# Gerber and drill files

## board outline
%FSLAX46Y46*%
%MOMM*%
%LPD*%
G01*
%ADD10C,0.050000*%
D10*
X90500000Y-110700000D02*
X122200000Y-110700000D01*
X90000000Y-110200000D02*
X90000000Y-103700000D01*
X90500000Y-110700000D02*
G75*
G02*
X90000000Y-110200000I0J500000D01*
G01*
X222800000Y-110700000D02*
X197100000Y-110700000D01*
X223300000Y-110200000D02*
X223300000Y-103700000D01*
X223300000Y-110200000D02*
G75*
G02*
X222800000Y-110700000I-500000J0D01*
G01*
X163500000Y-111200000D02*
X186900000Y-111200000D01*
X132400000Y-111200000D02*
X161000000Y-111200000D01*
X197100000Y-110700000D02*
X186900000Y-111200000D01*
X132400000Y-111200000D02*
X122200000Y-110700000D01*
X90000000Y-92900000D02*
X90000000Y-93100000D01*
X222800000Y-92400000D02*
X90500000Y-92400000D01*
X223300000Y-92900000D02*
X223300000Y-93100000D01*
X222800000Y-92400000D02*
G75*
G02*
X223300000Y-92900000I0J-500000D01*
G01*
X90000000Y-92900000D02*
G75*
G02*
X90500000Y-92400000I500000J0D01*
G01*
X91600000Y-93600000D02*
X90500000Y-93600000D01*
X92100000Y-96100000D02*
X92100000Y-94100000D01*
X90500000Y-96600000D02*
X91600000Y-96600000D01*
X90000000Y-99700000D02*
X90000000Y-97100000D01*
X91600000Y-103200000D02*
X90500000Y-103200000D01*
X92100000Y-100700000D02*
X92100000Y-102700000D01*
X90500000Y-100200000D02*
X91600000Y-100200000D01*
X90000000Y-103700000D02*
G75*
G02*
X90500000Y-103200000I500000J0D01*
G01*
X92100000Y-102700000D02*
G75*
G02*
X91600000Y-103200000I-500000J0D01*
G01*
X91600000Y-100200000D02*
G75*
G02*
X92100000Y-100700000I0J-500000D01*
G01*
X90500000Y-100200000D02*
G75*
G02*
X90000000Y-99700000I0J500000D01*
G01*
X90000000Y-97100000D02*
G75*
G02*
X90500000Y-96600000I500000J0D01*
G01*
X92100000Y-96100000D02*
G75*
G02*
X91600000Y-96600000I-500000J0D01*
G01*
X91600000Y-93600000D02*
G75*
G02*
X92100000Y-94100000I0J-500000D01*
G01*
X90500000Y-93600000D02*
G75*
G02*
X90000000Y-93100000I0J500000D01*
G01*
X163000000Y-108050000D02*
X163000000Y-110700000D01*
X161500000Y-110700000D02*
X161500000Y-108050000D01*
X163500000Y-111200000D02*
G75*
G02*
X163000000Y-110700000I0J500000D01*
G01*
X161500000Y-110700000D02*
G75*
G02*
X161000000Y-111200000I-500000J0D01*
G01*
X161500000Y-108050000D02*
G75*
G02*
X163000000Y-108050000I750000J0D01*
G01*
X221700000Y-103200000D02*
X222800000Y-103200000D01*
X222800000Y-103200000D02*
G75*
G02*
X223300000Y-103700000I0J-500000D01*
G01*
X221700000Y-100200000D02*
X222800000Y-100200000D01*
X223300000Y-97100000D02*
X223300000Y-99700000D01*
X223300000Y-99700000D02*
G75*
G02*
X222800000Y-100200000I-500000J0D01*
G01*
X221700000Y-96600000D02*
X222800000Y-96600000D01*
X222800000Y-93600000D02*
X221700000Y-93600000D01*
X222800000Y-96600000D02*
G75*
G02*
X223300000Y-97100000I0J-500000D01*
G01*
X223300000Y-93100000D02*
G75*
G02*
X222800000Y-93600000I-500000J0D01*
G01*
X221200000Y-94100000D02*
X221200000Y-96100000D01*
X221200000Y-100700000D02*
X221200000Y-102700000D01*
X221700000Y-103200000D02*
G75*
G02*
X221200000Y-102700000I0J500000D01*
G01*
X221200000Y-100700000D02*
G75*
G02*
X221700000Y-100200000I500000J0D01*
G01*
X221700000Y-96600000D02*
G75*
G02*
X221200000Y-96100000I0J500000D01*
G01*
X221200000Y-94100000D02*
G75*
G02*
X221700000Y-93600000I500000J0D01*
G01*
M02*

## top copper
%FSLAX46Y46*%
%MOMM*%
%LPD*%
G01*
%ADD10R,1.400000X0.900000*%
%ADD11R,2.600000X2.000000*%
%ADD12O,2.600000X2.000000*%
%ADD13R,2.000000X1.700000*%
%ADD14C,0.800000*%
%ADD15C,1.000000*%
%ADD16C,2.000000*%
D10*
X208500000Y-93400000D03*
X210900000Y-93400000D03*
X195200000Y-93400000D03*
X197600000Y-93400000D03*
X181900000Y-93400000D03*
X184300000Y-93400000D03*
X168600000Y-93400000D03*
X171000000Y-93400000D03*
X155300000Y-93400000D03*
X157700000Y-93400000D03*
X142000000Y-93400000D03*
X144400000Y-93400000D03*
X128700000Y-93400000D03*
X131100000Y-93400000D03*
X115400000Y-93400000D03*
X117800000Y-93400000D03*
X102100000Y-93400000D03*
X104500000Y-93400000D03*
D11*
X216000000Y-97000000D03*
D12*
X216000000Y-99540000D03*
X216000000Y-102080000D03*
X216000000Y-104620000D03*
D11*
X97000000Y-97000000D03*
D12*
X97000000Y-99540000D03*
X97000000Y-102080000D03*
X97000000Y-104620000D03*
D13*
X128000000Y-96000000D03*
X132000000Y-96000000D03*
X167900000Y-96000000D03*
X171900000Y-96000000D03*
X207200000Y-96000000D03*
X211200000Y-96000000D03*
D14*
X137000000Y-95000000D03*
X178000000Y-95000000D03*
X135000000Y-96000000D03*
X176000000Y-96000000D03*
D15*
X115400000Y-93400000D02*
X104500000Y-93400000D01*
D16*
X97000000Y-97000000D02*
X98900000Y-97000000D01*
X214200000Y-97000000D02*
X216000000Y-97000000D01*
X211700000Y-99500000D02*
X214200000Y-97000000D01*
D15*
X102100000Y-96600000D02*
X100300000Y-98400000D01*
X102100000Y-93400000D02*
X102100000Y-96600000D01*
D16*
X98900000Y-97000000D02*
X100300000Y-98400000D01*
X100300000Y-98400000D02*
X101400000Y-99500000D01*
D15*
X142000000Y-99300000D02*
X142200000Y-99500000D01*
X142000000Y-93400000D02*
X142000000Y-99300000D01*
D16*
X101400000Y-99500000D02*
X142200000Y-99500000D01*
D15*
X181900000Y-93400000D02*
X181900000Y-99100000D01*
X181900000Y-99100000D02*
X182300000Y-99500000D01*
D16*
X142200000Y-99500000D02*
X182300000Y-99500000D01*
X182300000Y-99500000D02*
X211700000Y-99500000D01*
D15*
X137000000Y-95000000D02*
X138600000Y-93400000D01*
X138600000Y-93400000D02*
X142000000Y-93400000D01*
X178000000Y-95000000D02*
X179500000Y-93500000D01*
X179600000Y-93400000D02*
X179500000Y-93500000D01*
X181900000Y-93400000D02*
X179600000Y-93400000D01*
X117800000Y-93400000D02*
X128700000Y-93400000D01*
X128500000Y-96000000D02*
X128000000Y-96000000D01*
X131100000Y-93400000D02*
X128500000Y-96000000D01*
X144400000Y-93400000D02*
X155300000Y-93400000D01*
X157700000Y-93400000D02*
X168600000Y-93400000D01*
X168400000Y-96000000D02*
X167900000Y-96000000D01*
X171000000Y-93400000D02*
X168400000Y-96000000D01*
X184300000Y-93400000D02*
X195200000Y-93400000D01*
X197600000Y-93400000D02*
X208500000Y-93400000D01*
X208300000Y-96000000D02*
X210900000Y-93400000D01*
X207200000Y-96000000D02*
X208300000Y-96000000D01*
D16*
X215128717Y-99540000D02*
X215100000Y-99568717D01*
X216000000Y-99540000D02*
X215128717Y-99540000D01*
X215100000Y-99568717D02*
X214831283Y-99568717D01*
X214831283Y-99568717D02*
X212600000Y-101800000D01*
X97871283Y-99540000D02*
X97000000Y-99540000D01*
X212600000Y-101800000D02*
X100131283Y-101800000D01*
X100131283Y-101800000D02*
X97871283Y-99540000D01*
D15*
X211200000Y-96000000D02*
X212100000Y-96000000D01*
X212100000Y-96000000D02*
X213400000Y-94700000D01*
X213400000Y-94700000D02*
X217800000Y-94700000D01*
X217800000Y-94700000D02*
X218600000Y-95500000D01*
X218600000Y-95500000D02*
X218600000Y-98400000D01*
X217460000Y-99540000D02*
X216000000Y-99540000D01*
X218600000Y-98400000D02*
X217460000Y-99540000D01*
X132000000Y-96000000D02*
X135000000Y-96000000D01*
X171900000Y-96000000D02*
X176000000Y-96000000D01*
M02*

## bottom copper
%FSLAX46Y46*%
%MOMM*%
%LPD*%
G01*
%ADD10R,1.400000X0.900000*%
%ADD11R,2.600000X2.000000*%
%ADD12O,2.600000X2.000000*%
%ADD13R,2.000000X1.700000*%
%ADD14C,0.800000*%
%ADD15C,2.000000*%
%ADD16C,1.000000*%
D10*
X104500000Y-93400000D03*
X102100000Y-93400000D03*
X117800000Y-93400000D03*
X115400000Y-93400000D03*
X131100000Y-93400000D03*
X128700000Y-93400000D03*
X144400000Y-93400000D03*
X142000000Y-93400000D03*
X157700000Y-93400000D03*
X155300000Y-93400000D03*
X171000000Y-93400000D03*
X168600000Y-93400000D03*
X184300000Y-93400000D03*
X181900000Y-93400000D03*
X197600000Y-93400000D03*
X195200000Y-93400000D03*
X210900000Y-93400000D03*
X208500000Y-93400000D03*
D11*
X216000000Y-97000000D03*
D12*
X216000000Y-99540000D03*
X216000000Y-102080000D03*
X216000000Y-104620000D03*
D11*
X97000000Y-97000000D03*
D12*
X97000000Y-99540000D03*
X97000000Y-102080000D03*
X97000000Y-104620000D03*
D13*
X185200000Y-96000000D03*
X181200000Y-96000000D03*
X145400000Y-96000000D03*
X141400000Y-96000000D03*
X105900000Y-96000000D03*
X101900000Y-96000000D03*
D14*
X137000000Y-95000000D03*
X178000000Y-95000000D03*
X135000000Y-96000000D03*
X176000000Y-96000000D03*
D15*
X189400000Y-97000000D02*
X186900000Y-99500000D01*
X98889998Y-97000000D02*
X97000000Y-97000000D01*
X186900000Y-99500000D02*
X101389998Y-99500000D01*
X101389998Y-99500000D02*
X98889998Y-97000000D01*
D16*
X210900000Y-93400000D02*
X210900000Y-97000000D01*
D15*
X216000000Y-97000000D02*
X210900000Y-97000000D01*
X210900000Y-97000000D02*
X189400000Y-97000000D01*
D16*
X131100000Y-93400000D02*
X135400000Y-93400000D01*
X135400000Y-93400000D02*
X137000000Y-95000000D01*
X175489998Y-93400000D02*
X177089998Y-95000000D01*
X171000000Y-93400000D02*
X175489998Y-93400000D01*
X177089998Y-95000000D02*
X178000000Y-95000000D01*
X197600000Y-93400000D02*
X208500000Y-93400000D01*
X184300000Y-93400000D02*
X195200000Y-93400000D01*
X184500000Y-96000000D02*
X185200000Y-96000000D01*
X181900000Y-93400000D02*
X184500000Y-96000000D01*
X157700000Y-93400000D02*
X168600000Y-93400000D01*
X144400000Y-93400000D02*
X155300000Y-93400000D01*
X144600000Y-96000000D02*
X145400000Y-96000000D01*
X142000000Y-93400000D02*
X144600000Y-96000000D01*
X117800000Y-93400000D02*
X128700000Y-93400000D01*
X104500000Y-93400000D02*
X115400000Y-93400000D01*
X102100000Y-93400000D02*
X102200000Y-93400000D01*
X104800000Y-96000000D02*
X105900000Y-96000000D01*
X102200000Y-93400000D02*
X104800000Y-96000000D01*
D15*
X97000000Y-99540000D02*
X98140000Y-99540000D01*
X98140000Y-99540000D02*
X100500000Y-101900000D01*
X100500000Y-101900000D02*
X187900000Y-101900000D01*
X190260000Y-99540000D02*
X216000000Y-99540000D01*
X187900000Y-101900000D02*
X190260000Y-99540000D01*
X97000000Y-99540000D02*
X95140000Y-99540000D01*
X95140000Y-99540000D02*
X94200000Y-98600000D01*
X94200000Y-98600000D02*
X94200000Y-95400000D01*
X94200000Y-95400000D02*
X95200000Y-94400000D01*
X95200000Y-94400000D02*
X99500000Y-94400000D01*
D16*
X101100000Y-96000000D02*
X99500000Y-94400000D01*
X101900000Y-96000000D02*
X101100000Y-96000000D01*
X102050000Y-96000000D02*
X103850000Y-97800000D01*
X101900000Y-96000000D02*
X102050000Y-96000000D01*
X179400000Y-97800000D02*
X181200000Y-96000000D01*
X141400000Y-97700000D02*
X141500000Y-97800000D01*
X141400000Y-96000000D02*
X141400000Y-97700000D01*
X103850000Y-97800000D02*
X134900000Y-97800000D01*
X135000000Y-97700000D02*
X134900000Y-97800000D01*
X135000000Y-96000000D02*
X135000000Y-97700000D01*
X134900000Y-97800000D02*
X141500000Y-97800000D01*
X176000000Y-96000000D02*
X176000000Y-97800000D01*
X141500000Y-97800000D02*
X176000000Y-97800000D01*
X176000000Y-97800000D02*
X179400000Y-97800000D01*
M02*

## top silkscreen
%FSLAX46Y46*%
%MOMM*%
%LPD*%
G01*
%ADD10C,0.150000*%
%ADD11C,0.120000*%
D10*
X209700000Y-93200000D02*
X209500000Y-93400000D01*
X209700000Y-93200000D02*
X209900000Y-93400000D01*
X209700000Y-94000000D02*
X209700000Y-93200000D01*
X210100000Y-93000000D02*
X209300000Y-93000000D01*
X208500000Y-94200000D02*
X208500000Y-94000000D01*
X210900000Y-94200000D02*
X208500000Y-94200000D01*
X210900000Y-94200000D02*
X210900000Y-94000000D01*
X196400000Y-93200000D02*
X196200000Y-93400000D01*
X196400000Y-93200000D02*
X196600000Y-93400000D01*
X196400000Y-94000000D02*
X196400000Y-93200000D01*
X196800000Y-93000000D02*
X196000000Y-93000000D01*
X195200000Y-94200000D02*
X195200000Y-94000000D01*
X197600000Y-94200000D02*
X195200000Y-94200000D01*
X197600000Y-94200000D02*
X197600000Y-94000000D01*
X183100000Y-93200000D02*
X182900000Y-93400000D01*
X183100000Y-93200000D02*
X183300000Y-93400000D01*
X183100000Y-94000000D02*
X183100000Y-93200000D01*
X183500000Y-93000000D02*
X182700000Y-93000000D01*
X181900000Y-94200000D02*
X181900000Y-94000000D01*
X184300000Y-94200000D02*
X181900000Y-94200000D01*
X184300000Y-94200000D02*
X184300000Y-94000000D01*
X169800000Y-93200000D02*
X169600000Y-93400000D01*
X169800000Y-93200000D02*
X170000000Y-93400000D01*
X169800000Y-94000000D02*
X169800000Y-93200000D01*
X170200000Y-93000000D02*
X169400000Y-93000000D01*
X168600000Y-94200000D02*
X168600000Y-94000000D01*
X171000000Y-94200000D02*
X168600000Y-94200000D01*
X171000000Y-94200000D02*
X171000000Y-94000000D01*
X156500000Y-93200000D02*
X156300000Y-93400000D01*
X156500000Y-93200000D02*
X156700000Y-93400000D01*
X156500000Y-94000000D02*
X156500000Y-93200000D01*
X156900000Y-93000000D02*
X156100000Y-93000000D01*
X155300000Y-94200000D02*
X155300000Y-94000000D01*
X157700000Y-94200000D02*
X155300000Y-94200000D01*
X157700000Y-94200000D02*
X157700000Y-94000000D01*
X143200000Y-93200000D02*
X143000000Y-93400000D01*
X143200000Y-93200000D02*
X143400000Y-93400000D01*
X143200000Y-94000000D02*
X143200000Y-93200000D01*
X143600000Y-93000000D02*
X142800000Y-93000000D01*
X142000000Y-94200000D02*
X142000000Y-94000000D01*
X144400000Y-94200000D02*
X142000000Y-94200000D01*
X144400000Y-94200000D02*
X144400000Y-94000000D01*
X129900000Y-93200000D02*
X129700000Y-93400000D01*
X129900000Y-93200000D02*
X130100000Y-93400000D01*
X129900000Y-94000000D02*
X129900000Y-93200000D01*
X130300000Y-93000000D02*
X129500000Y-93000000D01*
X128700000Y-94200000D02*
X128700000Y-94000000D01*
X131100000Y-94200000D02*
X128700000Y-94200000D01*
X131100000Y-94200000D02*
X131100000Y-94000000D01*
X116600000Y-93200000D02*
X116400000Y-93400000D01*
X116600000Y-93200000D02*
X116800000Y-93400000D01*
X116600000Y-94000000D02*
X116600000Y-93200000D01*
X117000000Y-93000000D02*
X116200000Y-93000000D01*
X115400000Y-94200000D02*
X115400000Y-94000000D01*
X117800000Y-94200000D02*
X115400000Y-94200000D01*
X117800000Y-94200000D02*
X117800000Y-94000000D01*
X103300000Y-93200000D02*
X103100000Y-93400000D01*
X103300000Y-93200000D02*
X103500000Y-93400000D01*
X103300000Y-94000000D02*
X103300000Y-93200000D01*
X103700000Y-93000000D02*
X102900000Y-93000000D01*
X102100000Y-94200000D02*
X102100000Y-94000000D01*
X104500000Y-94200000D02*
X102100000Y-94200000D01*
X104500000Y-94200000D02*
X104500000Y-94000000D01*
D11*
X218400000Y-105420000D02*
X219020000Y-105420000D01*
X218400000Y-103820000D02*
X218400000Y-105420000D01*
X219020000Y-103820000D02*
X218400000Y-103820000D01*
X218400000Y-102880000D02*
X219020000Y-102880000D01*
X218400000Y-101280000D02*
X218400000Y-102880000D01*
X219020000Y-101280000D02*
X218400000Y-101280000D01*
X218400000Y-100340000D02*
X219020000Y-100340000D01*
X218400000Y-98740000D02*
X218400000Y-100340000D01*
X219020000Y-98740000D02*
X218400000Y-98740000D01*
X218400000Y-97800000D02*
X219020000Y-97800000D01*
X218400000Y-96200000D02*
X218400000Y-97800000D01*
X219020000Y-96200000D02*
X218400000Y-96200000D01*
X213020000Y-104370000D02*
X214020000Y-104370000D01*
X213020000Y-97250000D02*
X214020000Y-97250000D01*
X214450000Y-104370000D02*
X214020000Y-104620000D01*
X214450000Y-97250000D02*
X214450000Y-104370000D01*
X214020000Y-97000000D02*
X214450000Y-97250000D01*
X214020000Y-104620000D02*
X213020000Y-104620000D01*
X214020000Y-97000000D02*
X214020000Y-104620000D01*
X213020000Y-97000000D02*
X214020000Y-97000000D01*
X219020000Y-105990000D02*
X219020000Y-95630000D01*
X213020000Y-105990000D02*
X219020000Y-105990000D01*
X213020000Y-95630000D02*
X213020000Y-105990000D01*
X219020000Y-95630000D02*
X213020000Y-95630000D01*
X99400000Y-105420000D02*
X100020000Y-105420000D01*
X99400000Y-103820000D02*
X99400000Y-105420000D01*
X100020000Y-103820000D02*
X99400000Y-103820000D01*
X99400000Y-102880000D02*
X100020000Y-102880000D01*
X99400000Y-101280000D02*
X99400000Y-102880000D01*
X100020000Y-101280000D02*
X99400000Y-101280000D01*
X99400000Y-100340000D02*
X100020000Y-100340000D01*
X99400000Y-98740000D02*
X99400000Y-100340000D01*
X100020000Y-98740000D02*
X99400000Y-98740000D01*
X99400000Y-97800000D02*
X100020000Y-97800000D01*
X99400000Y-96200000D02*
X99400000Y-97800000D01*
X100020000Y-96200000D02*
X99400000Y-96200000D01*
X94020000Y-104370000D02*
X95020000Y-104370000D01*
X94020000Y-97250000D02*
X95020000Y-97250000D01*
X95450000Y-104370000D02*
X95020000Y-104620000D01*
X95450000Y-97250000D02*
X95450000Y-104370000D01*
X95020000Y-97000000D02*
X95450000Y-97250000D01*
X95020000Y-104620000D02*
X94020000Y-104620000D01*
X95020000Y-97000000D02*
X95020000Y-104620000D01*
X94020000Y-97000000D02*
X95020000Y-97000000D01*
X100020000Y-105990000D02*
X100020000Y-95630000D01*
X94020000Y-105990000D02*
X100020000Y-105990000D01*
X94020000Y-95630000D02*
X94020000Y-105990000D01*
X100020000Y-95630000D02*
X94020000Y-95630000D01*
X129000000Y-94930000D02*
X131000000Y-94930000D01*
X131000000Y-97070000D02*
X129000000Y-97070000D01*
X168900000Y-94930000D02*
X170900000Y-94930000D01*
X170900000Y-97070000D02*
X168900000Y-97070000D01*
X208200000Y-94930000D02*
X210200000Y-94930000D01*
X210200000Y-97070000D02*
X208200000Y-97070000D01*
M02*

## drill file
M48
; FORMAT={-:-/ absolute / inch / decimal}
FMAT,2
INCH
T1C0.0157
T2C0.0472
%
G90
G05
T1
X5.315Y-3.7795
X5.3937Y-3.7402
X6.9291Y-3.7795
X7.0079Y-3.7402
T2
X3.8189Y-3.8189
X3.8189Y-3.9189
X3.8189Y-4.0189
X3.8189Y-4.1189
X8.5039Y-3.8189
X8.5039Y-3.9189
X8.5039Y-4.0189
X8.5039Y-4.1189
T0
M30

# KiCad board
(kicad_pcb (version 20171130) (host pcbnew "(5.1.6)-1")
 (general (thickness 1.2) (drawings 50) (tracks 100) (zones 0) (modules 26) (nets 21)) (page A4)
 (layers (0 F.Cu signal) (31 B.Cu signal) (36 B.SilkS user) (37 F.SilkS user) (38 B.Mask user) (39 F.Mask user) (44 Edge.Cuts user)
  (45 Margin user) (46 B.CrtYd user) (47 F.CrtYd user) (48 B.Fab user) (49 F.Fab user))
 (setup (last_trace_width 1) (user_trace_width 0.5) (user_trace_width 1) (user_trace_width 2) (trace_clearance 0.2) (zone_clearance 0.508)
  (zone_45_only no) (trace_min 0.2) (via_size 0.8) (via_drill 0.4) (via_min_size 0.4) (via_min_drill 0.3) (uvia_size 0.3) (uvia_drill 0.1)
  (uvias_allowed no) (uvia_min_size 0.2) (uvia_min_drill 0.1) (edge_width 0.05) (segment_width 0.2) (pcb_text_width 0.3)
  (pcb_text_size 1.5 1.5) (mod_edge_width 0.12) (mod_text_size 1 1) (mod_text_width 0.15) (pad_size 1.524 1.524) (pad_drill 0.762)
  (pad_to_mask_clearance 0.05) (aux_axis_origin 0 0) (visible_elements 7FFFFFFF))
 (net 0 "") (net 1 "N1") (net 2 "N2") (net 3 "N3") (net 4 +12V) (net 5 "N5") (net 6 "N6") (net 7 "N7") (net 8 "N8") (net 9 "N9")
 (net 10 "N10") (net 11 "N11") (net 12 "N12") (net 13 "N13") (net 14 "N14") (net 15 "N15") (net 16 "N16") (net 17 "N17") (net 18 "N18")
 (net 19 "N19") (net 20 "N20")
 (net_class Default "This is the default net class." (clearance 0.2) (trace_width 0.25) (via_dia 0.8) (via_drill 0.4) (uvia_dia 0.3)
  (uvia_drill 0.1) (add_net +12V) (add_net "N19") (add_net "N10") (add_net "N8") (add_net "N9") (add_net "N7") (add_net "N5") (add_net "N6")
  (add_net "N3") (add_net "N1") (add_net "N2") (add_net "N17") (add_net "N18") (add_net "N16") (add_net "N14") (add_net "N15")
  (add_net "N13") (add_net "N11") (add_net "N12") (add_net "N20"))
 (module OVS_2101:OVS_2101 (layer B.Cu) (at 103.3 93.4)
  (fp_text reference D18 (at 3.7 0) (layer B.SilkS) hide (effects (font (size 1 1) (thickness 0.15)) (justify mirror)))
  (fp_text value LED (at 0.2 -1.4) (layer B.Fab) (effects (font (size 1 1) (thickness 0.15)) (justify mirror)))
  (pad 2 smd rect (at 1.2 0) (size 1.4 0.9) (layers B.Cu B.Paste B.Mask) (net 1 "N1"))
  (pad 1 smd rect (at -1.2 0) (size 1.4 0.9) (layers B.Cu B.Paste B.Mask) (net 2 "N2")))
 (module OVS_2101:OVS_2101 (layer B.Cu) (at 116.6 93.4)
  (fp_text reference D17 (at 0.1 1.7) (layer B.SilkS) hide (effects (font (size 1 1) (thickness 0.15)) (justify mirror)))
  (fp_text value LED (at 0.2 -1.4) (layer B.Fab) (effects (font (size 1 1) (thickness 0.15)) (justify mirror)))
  (pad 2 smd rect (at 1.2 0) (size 1.4 0.9) (layers B.Cu B.Paste B.Mask) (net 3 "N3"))
  (pad 1 smd rect (at -1.2 0) (size 1.4 0.9) (layers B.Cu B.Paste B.Mask) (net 1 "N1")))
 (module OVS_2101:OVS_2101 (layer B.Cu) (at 129.9 93.4)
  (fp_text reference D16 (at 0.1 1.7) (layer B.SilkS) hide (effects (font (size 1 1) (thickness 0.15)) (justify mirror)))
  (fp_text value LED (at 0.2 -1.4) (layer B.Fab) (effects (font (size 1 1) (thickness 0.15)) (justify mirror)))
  (pad 2 smd rect (at 1.2 0) (size 1.4 0.9) (layers B.Cu B.Paste B.Mask) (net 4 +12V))
  (pad 1 smd rect (at -1.2 0) (size 1.4 0.9) (layers B.Cu B.Paste B.Mask) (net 3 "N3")))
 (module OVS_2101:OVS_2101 (layer B.Cu) (at 143.2 93.4)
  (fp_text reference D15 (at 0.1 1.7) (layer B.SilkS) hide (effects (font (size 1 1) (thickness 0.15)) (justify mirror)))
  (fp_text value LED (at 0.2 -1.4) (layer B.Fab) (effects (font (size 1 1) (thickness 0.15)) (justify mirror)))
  (pad 2 smd rect (at 1.2 0) (size 1.4 0.9) (layers B.Cu B.Paste B.Mask) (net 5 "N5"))
  (pad 1 smd rect (at -1.2 0) (size 1.4 0.9) (layers B.Cu B.Paste B.Mask) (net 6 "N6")))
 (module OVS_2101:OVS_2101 (layer B.Cu) (at 156.5 93.4)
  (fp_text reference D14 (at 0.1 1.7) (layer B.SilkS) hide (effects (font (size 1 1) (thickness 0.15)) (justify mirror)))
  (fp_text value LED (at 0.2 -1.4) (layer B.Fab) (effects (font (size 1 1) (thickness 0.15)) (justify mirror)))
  (pad 2 smd rect (at 1.2 0) (size 1.4 0.9) (layers B.Cu B.Paste B.Mask) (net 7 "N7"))
  (pad 1 smd rect (at -1.2 0) (size 1.4 0.9) (layers B.Cu B.Paste B.Mask) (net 5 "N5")))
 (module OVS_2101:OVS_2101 (layer B.Cu) (at 169.8 93.4)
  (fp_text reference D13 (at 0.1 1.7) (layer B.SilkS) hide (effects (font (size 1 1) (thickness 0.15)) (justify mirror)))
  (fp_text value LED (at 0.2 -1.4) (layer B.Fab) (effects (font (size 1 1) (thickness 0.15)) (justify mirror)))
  (pad 2 smd rect (at 1.2 0) (size 1.4 0.9) (layers B.Cu B.Paste B.Mask) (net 4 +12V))
  (pad 1 smd rect (at -1.2 0) (size 1.4 0.9) (layers B.Cu B.Paste B.Mask) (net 7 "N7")))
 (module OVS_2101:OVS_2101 (layer B.Cu) (at 183.1 93.4)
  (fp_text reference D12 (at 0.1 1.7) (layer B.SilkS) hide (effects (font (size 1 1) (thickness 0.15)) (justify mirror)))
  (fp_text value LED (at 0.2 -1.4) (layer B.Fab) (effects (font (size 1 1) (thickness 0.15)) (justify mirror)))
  (pad 2 smd rect (at 1.2 0) (size 1.4 0.9) (layers B.Cu B.Paste B.Mask) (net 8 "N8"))
  (pad 1 smd rect (at -1.2 0) (size 1.4 0.9) (layers B.Cu B.Paste B.Mask) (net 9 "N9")))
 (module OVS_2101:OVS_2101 (layer B.Cu) (at 196.4 93.4)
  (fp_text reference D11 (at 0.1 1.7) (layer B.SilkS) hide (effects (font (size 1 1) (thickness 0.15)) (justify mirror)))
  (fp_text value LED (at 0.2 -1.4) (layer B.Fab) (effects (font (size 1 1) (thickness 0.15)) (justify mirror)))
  (pad 2 smd rect (at 1.2 0) (size 1.4 0.9) (layers B.Cu B.Paste B.Mask) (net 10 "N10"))
  (pad 1 smd rect (at -1.2 0) (size 1.4 0.9) (layers B.Cu B.Paste B.Mask) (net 8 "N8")))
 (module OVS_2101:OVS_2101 (layer B.Cu) (at 209.7 93.4)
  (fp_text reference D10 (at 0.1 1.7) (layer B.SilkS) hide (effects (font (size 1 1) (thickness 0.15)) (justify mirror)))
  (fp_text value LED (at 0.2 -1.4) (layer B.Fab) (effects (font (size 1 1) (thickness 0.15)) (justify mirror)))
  (pad 2 smd rect (at 1.2 0) (size 1.4 0.9) (layers B.Cu B.Paste B.Mask) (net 4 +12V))
  (pad 1 smd rect (at -1.2 0) (size 1.4 0.9) (layers B.Cu B.Paste B.Mask) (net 10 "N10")))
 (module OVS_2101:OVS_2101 (layer F.Cu) (at 209.7 93.4 180)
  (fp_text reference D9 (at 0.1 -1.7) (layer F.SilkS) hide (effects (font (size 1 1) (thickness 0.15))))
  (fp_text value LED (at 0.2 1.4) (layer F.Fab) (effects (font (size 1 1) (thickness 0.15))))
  (fp_line (start 0 0.2) (end 0.2 0) (layer F.SilkS) (width 0.15))
  (fp_line (start 0 0.2) (end -0.2 0) (layer F.SilkS) (width 0.15))
  (fp_line (start 0 -0.6) (end 0 0.2) (layer F.SilkS) (width 0.15))
  (fp_line (start -0.4 0.4) (end 0.4 0.4) (layer F.SilkS) (width 0.15))
  (fp_line (start 1.2 -0.8) (end 1.2 -0.6) (layer F.SilkS) (width 0.15))
  (fp_line (start -1.2 -0.8) (end 1.2 -0.8) (layer F.SilkS) (width 0.15))
  (fp_line (start -1.2 -0.8) (end -1.2 -0.6) (layer F.SilkS) (width 0.15))
  (pad 2 smd rect (at 1.2 0 180) (size 1.4 0.9) (layers F.Cu F.Paste F.Mask) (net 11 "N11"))
  (pad 1 smd rect (at -1.2 0 180) (size 1.4 0.9) (layers F.Cu F.Paste F.Mask) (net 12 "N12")))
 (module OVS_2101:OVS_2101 (layer F.Cu) (at 196.4 93.4 180)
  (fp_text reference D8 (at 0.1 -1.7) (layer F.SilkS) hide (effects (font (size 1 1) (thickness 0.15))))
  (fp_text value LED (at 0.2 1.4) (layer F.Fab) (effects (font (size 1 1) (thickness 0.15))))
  (fp_line (start 0 0.2) (end 0.2 0) (layer F.SilkS) (width 0.15))
  (fp_line (start 0 0.2) (end -0.2 0) (layer F.SilkS) (width 0.15))
  (fp_line (start 0 -0.6) (end 0 0.2) (layer F.SilkS) (width 0.15))
  (fp_line (start -0.4 0.4) (end 0.4 0.4) (layer F.SilkS) (width 0.15))
  (fp_line (start 1.2 -0.8) (end 1.2 -0.6) (layer F.SilkS) (width 0.15))
  (fp_line (start -1.2 -0.8) (end 1.2 -0.8) (layer F.SilkS) (width 0.15))
  (fp_line (start -1.2 -0.8) (end -1.2 -0.6) (layer F.SilkS) (width 0.15))
  (pad 2 smd rect (at 1.2 0 180) (size 1.4 0.9) (layers F.Cu F.Paste F.Mask) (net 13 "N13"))
  (pad 1 smd rect (at -1.2 0 180) (size 1.4 0.9) (layers F.Cu F.Paste F.Mask) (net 11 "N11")))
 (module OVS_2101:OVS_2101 (layer F.Cu) (at 183.1 93.4 180)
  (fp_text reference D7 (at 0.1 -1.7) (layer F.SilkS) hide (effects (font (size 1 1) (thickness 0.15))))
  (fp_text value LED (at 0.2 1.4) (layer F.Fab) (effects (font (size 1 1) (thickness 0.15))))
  (fp_line (start 0 0.2) (end 0.2 0) (layer F.SilkS) (width 0.15))
  (fp_line (start 0 0.2) (end -0.2 0) (layer F.SilkS) (width 0.15))
  (fp_line (start 0 -0.6) (end 0 0.2) (layer F.SilkS) (width 0.15))
  (fp_line (start -0.4 0.4) (end 0.4 0.4) (layer F.SilkS) (width 0.15))
  (fp_line (start 1.2 -0.8) (end 1.2 -0.6) (layer F.SilkS) (width 0.15))
  (fp_line (start -1.2 -0.8) (end 1.2 -0.8) (layer F.SilkS) (width 0.15))
  (fp_line (start -1.2 -0.8) (end -1.2 -0.6) (layer F.SilkS) (width 0.15))
  (pad 2 smd rect (at 1.2 0 180) (size 1.4 0.9) (layers F.Cu F.Paste F.Mask) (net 4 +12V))
  (pad 1 smd rect (at -1.2 0 180) (size 1.4 0.9) (layers F.Cu F.Paste F.Mask) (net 13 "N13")))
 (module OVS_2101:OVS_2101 (layer F.Cu) (at 169.8 93.4 180)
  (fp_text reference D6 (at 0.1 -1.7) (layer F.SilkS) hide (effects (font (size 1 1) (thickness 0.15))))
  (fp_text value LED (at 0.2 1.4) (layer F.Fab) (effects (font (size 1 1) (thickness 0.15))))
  (fp_line (start 0 0.2) (end 0.2 0) (layer F.SilkS) (width 0.15))
  (fp_line (start 0 0.2) (end -0.2 0) (layer F.SilkS) (width 0.15))
  (fp_line (start 0 -0.6) (end 0 0.2) (layer F.SilkS) (width 0.15))
  (fp_line (start -0.4 0.4) (end 0.4 0.4) (layer F.SilkS) (width 0.15))
  (fp_line (start 1.2 -0.8) (end 1.2 -0.6) (layer F.SilkS) (width 0.15))
  (fp_line (start -1.2 -0.8) (end 1.2 -0.8) (layer F.SilkS) (width 0.15))
  (fp_line (start -1.2 -0.8) (end -1.2 -0.6) (layer F.SilkS) (width 0.15))
  (pad 2 smd rect (at 1.2 0 180) (size 1.4 0.9) (layers F.Cu F.Paste F.Mask) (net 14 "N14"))
  (pad 1 smd rect (at -1.2 0 180) (size 1.4 0.9) (layers F.Cu F.Paste F.Mask) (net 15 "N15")))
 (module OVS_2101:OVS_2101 (layer F.Cu) (at 156.5 93.4 180)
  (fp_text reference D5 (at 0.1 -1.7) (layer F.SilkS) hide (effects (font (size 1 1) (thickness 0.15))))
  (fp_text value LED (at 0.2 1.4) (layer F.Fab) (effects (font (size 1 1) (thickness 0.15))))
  (fp_line (start 0 0.2) (end 0.2 0) (layer F.SilkS) (width 0.15))
  (fp_line (start 0 0.2) (end -0.2 0) (layer F.SilkS) (width 0.15))
  (fp_line (start 0 -0.6) (end 0 0.2) (layer F.SilkS) (width 0.15))
  (fp_line (start -0.4 0.4) (end 0.4 0.4) (layer F.SilkS) (width 0.15))
  (fp_line (start 1.2 -0.8) (end 1.2 -0.6) (layer F.SilkS) (width 0.15))
  (fp_line (start -1.2 -0.8) (end 1.2 -0.8) (layer F.SilkS) (width 0.15))
  (fp_line (start -1.2 -0.8) (end -1.2 -0.6) (layer F.SilkS) (width 0.15))
  (pad 2 smd rect (at 1.2 0 180) (size 1.4 0.9) (layers F.Cu F.Paste F.Mask) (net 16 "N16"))
  (pad 1 smd rect (at -1.2 0 180) (size 1.4 0.9) (layers F.Cu F.Paste F.Mask) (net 14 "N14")))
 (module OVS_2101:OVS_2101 (layer F.Cu) (at 143.2 93.4 180)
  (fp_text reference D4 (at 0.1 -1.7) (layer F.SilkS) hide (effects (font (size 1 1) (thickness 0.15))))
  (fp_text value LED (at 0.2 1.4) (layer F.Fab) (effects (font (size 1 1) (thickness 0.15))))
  (fp_line (start 0 0.2) (end 0.2 0) (layer F.SilkS) (width 0.15))
  (fp_line (start 0 0.2) (end -0.2 0) (layer F.SilkS) (width 0.15))
  (fp_line (start 0 -0.6) (end 0 0.2) (layer F.SilkS) (width 0.15))
  (fp_line (start -0.4 0.4) (end 0.4 0.4) (layer F.SilkS) (width 0.15))
  (fp_line (start 1.2 -0.8) (end 1.2 -0.6) (layer F.SilkS) (width 0.15))
  (fp_line (start -1.2 -0.8) (end 1.2 -0.8) (layer F.SilkS) (width 0.15))
  (fp_line (start -1.2 -0.8) (end -1.2 -0.6) (layer F.SilkS) (width 0.15))
  (pad 2 smd rect (at 1.2 0 180) (size 1.4 0.9) (layers F.Cu F.Paste F.Mask) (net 4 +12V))
  (pad 1 smd rect (at -1.2 0 180) (size 1.4 0.9) (layers F.Cu F.Paste F.Mask) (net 16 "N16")))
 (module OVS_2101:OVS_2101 (layer F.Cu) (at 129.9 93.4 180)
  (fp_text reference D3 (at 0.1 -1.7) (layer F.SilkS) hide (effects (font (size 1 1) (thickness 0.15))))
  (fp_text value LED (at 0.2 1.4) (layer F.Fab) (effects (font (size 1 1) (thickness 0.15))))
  (fp_line (start 0 0.2) (end 0.2 0) (layer F.SilkS) (width 0.15))
  (fp_line (start 0 0.2) (end -0.2 0) (layer F.SilkS) (width 0.15))
  (fp_line (start 0 -0.6) (end 0 0.2) (layer F.SilkS) (width 0.15))
  (fp_line (start -0.4 0.4) (end 0.4 0.4) (layer F.SilkS) (width 0.15))
  (fp_line (start 1.2 -0.8) (end 1.2 -0.6) (layer F.SilkS) (width 0.15))
  (fp_line (start -1.2 -0.8) (end 1.2 -0.8) (layer F.SilkS) (width 0.15))
  (fp_line (start -1.2 -0.8) (end -1.2 -0.6) (layer F.SilkS) (width 0.15))
  (pad 2 smd rect (at 1.2 0 180) (size 1.4 0.9) (layers F.Cu F.Paste F.Mask) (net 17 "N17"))
  (pad 1 smd rect (at -1.2 0 180) (size 1.4 0.9) (layers F.Cu F.Paste F.Mask) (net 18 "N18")))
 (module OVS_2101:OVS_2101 (layer F.Cu) (at 116.6 93.4 180)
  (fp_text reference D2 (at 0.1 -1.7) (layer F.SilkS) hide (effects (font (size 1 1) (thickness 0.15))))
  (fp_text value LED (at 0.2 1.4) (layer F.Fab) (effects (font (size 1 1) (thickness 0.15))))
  (fp_line (start 0 0.2) (end 0.2 0) (layer F.SilkS) (width 0.15))
  (fp_line (start 0 0.2) (end -0.2 0) (layer F.SilkS) (width 0.15))
  (fp_line (start 0 -0.6) (end 0 0.2) (layer F.SilkS) (width 0.15))
  (fp_line (start -0.4 0.4) (end 0.4 0.4) (layer F.SilkS) (width 0.15))
  (fp_line (start 1.2 -0.8) (end 1.2 -0.6) (layer F.SilkS) (width 0.15))
  (fp_line (start -1.2 -0.8) (end 1.2 -0.8) (layer F.SilkS) (width 0.15))
  (fp_line (start -1.2 -0.8) (end -1.2 -0.6) (layer F.SilkS) (width 0.15))
  (pad 2 smd rect (at 1.2 0 180) (size 1.4 0.9) (layers F.Cu F.Paste F.Mask) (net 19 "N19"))
  (pad 1 smd rect (at -1.2 0 180) (size 1.4 0.9) (layers F.Cu F.Paste F.Mask) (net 17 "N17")))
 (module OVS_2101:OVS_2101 (layer F.Cu) (at 103.3 93.4 180)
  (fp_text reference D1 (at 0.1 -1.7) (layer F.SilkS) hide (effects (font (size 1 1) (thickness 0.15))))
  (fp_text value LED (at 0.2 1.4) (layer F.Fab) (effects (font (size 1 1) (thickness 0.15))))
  (fp_line (start 0 0.2) (end 0.2 0) (layer F.SilkS) (width 0.15))
  (fp_line (start 0 0.2) (end -0.2 0) (layer F.SilkS) (width 0.15))
  (fp_line (start 0 -0.6) (end 0 0.2) (layer F.SilkS) (width 0.15))
  (fp_line (start -0.4 0.4) (end 0.4 0.4) (layer F.SilkS) (width 0.15))
  (fp_line (start 1.2 -0.8) (end 1.2 -0.6) (layer F.SilkS) (width 0.15))
  (fp_line (start -1.2 -0.8) (end 1.2 -0.8) (layer F.SilkS) (width 0.15))
  (fp_line (start -1.2 -0.8) (end -1.2 -0.6) (layer F.SilkS) (width 0.15))
  (pad 2 smd rect (at 1.2 0 180) (size 1.4 0.9) (layers F.Cu F.Paste F.Mask) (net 4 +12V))
  (pad 1 smd rect (at -1.2 0 180) (size 1.4 0.9) (layers F.Cu F.Paste F.Mask) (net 19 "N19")))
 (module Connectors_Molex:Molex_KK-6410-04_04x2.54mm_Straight (layer F.Cu) (at 216 97 270)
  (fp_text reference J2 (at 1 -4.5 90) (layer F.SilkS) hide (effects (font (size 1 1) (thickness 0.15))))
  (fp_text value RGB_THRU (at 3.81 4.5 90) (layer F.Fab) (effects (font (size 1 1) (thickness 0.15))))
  (fp_line (start 8.42 -2.4) (end 8.42 -3.02) (layer F.SilkS) (width 0.12))
  (fp_line (start 6.82 -2.4) (end 8.42 -2.4) (layer F.SilkS) (width 0.12))
  (fp_line (start 6.82 -3.02) (end 6.82 -2.4) (layer F.SilkS) (width 0.12))
  (fp_line (start 5.88 -2.4) (end 5.88 -3.02) (layer F.SilkS) (width 0.12))
  (fp_line (start 4.28 -2.4) (end 5.88 -2.4) (layer F.SilkS) (width 0.12))
  (fp_line (start 4.28 -3.02) (end 4.28 -2.4) (layer F.SilkS) (width 0.12))
  (fp_line (start 3.34 -2.4) (end 3.34 -3.02) (layer F.SilkS) (width 0.12))
  (fp_line (start 1.74 -2.4) (end 3.34 -2.4) (layer F.SilkS) (width 0.12))
  (fp_line (start 1.74 -3.02) (end 1.74 -2.4) (layer F.SilkS) (width 0.12))
  (fp_line (start 0.8 -2.4) (end 0.8 -3.02) (layer F.SilkS) (width 0.12))
  (fp_line (start -0.8 -2.4) (end 0.8 -2.4) (layer F.SilkS) (width 0.12))
  (fp_line (start -0.8 -3.02) (end -0.8 -2.4) (layer F.SilkS) (width 0.12))
  (fp_line (start 7.37 2.98) (end 7.37 1.98) (layer F.SilkS) (width 0.12))
  (fp_line (start 0.25 2.98) (end 0.25 1.98) (layer F.SilkS) (width 0.12))
  (fp_line (start 7.37 1.55) (end 7.62 1.98) (layer F.SilkS) (width 0.12))
  (fp_line (start 0.25 1.55) (end 7.37 1.55) (layer F.SilkS) (width 0.12))
  (fp_line (start 0 1.98) (end 0.25 1.55) (layer F.SilkS) (width 0.12))
  (fp_line (start 7.62 1.98) (end 7.62 2.98) (layer F.SilkS) (width 0.12))
  (fp_line (start 0 1.98) (end 7.62 1.98) (layer F.SilkS) (width 0.12))
  (fp_line (start 0 2.98) (end 0 1.98) (layer F.SilkS) (width 0.12))
  (fp_line (start 8.99 -3.02) (end -1.37 -3.02) (layer F.SilkS) (width 0.12))
  (fp_line (start 8.99 2.98) (end 8.99 -3.02) (layer F.SilkS) (width 0.12))
  (fp_line (start -1.37 2.98) (end 8.99 2.98) (layer F.SilkS) (width 0.12))
  (fp_line (start -1.37 -3.02) (end -1.37 2.98) (layer F.SilkS) (width 0.12))
  (pad 1 thru_hole rect (at 0 0 270) (size 2 2.6) (drill 1.2) (layers *.Cu *.Mask) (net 4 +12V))
  (pad 2 thru_hole oval (at 2.54 0 270) (size 2 2.6) (drill 1.2) (layers *.Cu *.Mask) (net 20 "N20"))
  (pad 3 thru_hole oval (at 5.08 0 270) (size 2 2.6) (drill 1.2) (layers *.Cu *.Mask))
  (pad 4 thru_hole oval (at 7.62 0 270) (size 2 2.6) (drill 1.2) (layers *.Cu *.Mask)))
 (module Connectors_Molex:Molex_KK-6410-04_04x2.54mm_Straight (layer F.Cu) (at 97 97 270)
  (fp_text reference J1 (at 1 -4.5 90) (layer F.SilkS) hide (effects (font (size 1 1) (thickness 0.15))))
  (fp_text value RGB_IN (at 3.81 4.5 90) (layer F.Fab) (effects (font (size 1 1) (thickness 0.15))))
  (fp_line (start 8.42 -2.4) (end 8.42 -3.02) (layer F.SilkS) (width 0.12))
  (fp_line (start 6.82 -2.4) (end 8.42 -2.4) (layer F.SilkS) (width 0.12))
  (fp_line (start 6.82 -3.02) (end 6.82 -2.4) (layer F.SilkS) (width 0.12))
  (fp_line (start 5.88 -2.4) (end 5.88 -3.02) (layer F.SilkS) (width 0.12))
  (fp_line (start 4.28 -2.4) (end 5.88 -2.4) (layer F.SilkS) (width 0.12))
  (fp_line (start 4.28 -3.02) (end 4.28 -2.4) (layer F.SilkS) (width 0.12))
  (fp_line (start 3.34 -2.4) (end 3.34 -3.02) (layer F.SilkS) (width 0.12))
  (fp_line (start 1.74 -2.4) (end 3.34 -2.4) (layer F.SilkS) (width 0.12))
  (fp_line (start 1.74 -3.02) (end 1.74 -2.4) (layer F.SilkS) (width 0.12))
  (fp_line (start 0.8 -2.4) (end 0.8 -3.02) (layer F.SilkS) (width 0.12))
  (fp_line (start -0.8 -2.4) (end 0.8 -2.4) (layer F.SilkS) (width 0.12))
  (fp_line (start -0.8 -3.02) (end -0.8 -2.4) (layer F.SilkS) (width 0.12))
  (fp_line (start 7.37 2.98) (end 7.37 1.98) (layer F.SilkS) (width 0.12))
  (fp_line (start 0.25 2.98) (end 0.25 1.98) (layer F.SilkS) (width 0.12))
  (fp_line (start 7.37 1.55) (end 7.62 1.98) (layer F.SilkS) (width 0.12))
  (fp_line (start 0.25 1.55) (end 7.37 1.55) (layer F.SilkS) (width 0.12))
  (fp_line (start 0 1.98) (end 0.25 1.55) (layer F.SilkS) (width 0.12))
  (fp_line (start 7.62 1.98) (end 7.62 2.98) (layer F.SilkS) (width 0.12))
  (fp_line (start 0 1.98) (end 7.62 1.98) (layer F.SilkS) (width 0.12))
  (fp_line (start 0 2.98) (end 0 1.98) (layer F.SilkS) (width 0.12))
  (fp_line (start 8.99 -3.02) (end -1.37 -3.02) (layer F.SilkS) (width 0.12))
  (fp_line (start 8.99 2.98) (end 8.99 -3.02) (layer F.SilkS) (width 0.12))
  (fp_line (start -1.37 2.98) (end 8.99 2.98) (layer F.SilkS) (width 0.12))
  (fp_line (start -1.37 -3.02) (end -1.37 2.98) (layer F.SilkS) (width 0.12))
  (pad 1 thru_hole rect (at 0 0 270) (size 2 2.6) (drill 1.2) (layers *.Cu *.Mask) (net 4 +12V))
  (pad 2 thru_hole oval (at 2.54 0 270) (size 2 2.6) (drill 1.2) (layers *.Cu *.Mask) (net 20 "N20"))
  (pad 3 thru_hole oval (at 5.08 0 270) (size 2 2.6) (drill 1.2) (layers *.Cu *.Mask))
  (pad 4 thru_hole oval (at 7.62 0 270) (size 2 2.6) (drill 1.2) (layers *.Cu *.Mask)))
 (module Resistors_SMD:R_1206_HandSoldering (layer F.Cu) (at 130 96)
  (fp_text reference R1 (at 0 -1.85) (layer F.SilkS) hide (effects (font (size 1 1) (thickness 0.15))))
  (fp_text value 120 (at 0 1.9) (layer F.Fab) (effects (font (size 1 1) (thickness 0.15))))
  (fp_line (start -1 -1.07) (end 1 -1.07) (layer F.SilkS) (width 0.12))
  (fp_line (start 1 1.07) (end -1 1.07) (layer F.SilkS) (width 0.12))
  (pad 1 smd rect (at -2 0) (size 2 1.7) (layers F.Cu F.Paste F.Mask) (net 18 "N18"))
  (pad 2 smd rect (at 2 0) (size 2 1.7) (layers F.Cu F.Paste F.Mask) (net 20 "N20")))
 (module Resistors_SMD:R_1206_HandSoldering (layer F.Cu) (at 169.9 96)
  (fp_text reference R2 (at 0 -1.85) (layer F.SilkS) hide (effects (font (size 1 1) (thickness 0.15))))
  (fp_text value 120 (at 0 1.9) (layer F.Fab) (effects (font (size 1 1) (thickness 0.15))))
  (fp_line (start -1 -1.07) (end 1 -1.07) (layer F.SilkS) (width 0.12))
  (fp_line (start 1 1.07) (end -1 1.07) (layer F.SilkS) (width 0.12))
  (pad 1 smd rect (at -2 0) (size 2 1.7) (layers F.Cu F.Paste F.Mask) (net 15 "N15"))
  (pad 2 smd rect (at 2 0) (size 2 1.7) (layers F.Cu F.Paste F.Mask) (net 20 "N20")))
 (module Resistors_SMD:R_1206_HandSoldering (layer F.Cu) (at 209.2 96)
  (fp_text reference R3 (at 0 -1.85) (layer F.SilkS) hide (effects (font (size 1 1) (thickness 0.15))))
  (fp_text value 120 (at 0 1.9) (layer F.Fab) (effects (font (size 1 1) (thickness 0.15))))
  (fp_line (start -1 -1.07) (end 1 -1.07) (layer F.SilkS) (width 0.12))
  (fp_line (start 1 1.07) (end -1 1.07) (layer F.SilkS) (width 0.12))
  (pad 1 smd rect (at -2 0) (size 2 1.7) (layers F.Cu F.Paste F.Mask) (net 12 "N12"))
  (pad 2 smd rect (at 2 0) (size 2 1.7) (layers F.Cu F.Paste F.Mask) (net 20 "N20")))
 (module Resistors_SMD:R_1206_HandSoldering (layer B.Cu) (at 183.2 96 180)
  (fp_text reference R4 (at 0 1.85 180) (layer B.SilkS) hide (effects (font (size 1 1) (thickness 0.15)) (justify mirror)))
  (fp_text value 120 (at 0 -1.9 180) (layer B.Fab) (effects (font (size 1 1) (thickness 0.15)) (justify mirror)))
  (pad 1 smd rect (at -2 0 180) (size 2 1.7) (layers B.Cu B.Paste B.Mask) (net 9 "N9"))
  (pad 2 smd rect (at 2 0 180) (size 2 1.7) (layers B.Cu B.Paste B.Mask) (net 20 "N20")))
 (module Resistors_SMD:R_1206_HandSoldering (layer B.Cu) (at 143.4 96 180)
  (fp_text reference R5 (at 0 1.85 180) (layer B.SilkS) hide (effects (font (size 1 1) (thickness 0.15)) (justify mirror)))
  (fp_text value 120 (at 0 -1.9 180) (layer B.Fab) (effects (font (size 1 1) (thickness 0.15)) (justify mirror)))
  (pad 1 smd rect (at -2 0 180) (size 2 1.7) (layers B.Cu B.Paste B.Mask) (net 6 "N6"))
  (pad 2 smd rect (at 2 0 180) (size 2 1.7) (layers B.Cu B.Paste B.Mask) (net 20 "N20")))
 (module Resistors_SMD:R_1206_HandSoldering (layer B.Cu) (at 103.9 96 180)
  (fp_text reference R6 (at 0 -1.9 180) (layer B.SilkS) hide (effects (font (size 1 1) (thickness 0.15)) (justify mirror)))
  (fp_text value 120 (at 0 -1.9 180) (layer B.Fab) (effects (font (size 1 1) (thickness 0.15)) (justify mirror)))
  (pad 1 smd rect (at -2 0 180) (size 2 1.7) (layers B.Cu B.Paste B.Mask) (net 2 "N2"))
  (pad 2 smd rect (at 2 0 180) (size 2 1.7) (layers B.Cu B.Paste B.Mask) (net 20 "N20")))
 (gr_line (start 90.5 110.7) (end 122.2 110.7) (layer Edge.Cuts) (width 0.05))
 (gr_line (start 90 110.2) (end 90 103.7) (layer Edge.Cuts) (width 0.05))
 (gr_arc (start 90.5 110.2) (end 90 110.2) (angle -90) (layer Edge.Cuts) (width 0.05))
 (gr_line (start 222.8 110.7) (end 197.1 110.7) (layer Edge.Cuts) (width 0.05))
 (gr_line (start 223.3 110.2) (end 223.3 103.7) (layer Edge.Cuts) (width 0.05))
 (gr_arc (start 222.8 110.2) (end 222.8 110.7) (angle -90) (layer Edge.Cuts) (width 0.05))
 (gr_line (start 163.5 111.2) (end 186.9 111.2) (layer Edge.Cuts) (width 0.05))
 (gr_line (start 132.4 111.2) (end 161 111.2) (layer Edge.Cuts) (width 0.05))
 (gr_line (start 197.1 110.7) (end 186.9 111.2) (layer Edge.Cuts) (width 0.05))
 (gr_line (start 132.4 111.2) (end 122.2 110.7) (layer Edge.Cuts) (width 0.05))
 (gr_line (start 90 92.9) (end 90 93.1) (layer Edge.Cuts) (width 0.05))
 (gr_line (start 222.8 92.4) (end 90.5 92.4) (layer Edge.Cuts) (width 0.05))
 (gr_line (start 223.3 92.9) (end 223.3 93.1) (layer Edge.Cuts) (width 0.05))
 (gr_arc (start 222.8 92.9) (end 223.3 92.9) (angle -90) (layer Edge.Cuts) (width 0.05))
 (gr_arc (start 90.5 92.9) (end 90.5 92.4) (angle -90) (layer Edge.Cuts) (width 0.05))
 (gr_line (start 91.6 93.6) (end 90.5 93.6) (layer Edge.Cuts) (width 0.05))
 (gr_line (start 92.1 96.1) (end 92.1 94.1) (layer Edge.Cuts) (width 0.05))
 (gr_line (start 90.5 96.6) (end 91.6 96.6) (layer Edge.Cuts) (width 0.05))
 (gr_line (start 90 99.7) (end 90 97.1) (layer Edge.Cuts) (width 0.05))
 (gr_line (start 91.6 103.2) (end 90.5 103.2) (layer Edge.Cuts) (width 0.05))
 (gr_line (start 92.1 100.7) (end 92.1 102.7) (layer Edge.Cuts) (width 0.05))
 (gr_line (start 90.5 100.2) (end 91.6 100.2) (layer Edge.Cuts) (width 0.05))
 (gr_arc (start 90.5 103.7) (end 90.5 103.2) (angle -90) (layer Edge.Cuts) (width 0.05))
 (gr_arc (start 91.6 102.7) (end 91.6 103.2) (angle -90) (layer Edge.Cuts) (width 0.05))
 (gr_arc (start 91.6 100.7) (end 92.1 100.7) (angle -90) (layer Edge.Cuts) (width 0.05))
 (gr_arc (start 90.5 99.7) (end 90 99.7) (angle -90) (layer Edge.Cuts) (width 0.05))
 (gr_arc (start 90.5 97.1) (end 90.5 96.6) (angle -90) (layer Edge.Cuts) (width 0.05))
 (gr_arc (start 91.6 96.1) (end 91.6 96.6) (angle -90) (layer Edge.Cuts) (width 0.05))
 (gr_arc (start 91.6 94.1) (end 92.1 94.1) (angle -90) (layer Edge.Cuts) (width 0.05))
 (gr_arc (start 90.5 93.1) (end 90 93.1) (angle -90) (layer Edge.Cuts) (width 0.05))
 (gr_line (start 163 108.05) (end 163 110.7) (layer Edge.Cuts) (width 0.05))
 (gr_line (start 161.5 110.7) (end 161.5 108.05) (layer Edge.Cuts) (width 0.05))
 (gr_arc (start 163.5 110.7) (end 163 110.7) (angle -90) (layer Edge.Cuts) (width 0.05))
 (gr_arc (start 161 110.7) (end 161 111.2) (angle -90) (layer Edge.Cuts) (width 0.05))
 (gr_arc (start 162.25 108.05) (end 163 108.05) (angle -180) (layer Edge.Cuts) (width 0.05))
 (gr_line (start 221.7 103.2) (end 222.8 103.2) (layer Edge.Cuts) (width 0.05))
 (gr_arc (start 222.8 103.7) (end 223.3 103.7) (angle -90) (layer Edge.Cuts) (width 0.05))
 (gr_line (start 221.7 100.2) (end 222.8 100.2) (layer Edge.Cuts) (width 0.05))
 (gr_line (start 223.3 97.1) (end 223.3 99.7) (layer Edge.Cuts) (width 0.05))
 (gr_arc (start 222.8 99.7) (end 222.8 100.2) (angle -90) (layer Edge.Cuts) (width 0.05))
 (gr_line (start 221.7 96.6) (end 222.8 96.6) (layer Edge.Cuts) (width 0.05))
 (gr_line (start 222.8 93.6) (end 221.7 93.6) (layer Edge.Cuts) (width 0.05))
 (gr_arc (start 222.8 97.1) (end 223.3 97.1) (angle -90) (layer Edge.Cuts) (width 0.05))
 (gr_arc (start 222.8 93.1) (end 222.8 93.6) (angle -90) (layer Edge.Cuts) (width 0.05))
 (gr_line (start 221.2 94.1) (end 221.2 96.1) (layer Edge.Cuts) (width 0.05))
 (gr_line (start 221.2 100.7) (end 221.2 102.7) (layer Edge.Cuts) (width 0.05))
 (gr_arc (start 221.7 102.7) (end 221.2 102.7) (angle -90) (layer Edge.Cuts) (width 0.05))
 (gr_arc (start 221.7 100.7) (end 221.7 100.2) (angle -90) (layer Edge.Cuts) (width 0.05))
 (gr_arc (start 221.7 96.1) (end 221.2 96.1) (angle -90) (layer Edge.Cuts) (width 0.05))
 (gr_arc (start 221.7 94.1) (end 221.7 93.6) (angle -90) (layer Edge.Cuts) (width 0.05))
 (segment (start 115.4 93.4) (end 104.5 93.4) (width 1) (layer F.Cu) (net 19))
 (segment (start 189.4 97) (end 186.9 99.5) (width 2) (layer B.Cu) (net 4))
 (segment (start 98.889998 97) (end 97 97) (width 2) (layer B.Cu) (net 4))
 (segment (start 186.9 99.5) (end 101.389998 99.5) (width 2) (layer B.Cu) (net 4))
 (segment (start 101.389998 99.5) (end 98.889998 97) (width 2) (layer B.Cu) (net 4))
 (segment (start 97 97) (end 98.9 97) (width 2) (layer F.Cu) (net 4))
 (segment (start 214.2 97) (end 216 97) (width 2) (layer F.Cu) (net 4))
 (segment (start 211.7 99.5) (end 214.2 97) (width 2) (layer F.Cu) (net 4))
 (segment (start 102.1 96.6) (end 100.3 98.4) (width 1) (layer F.Cu) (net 4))
 (segment (start 102.1 93.4) (end 102.1 96.6) (width 1) (layer F.Cu) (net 4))
 (segment (start 98.9 97) (end 100.3 98.4) (width 2) (layer F.Cu) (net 4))
 (segment (start 100.3 98.4) (end 101.4 99.5) (width 2) (layer F.Cu) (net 4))
 (segment (start 142 99.3) (end 142.2 99.5) (width 1) (layer F.Cu) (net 4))
 (segment (start 142 93.4) (end 142 99.3) (width 1) (layer F.Cu) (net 4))
 (segment (start 101.4 99.5) (end 142.2 99.5) (width 2) (layer F.Cu) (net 4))
 (segment (start 181.9 93.4) (end 181.9 99.1) (width 1) (layer F.Cu) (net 4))
 (segment (start 181.9 99.1) (end 182.3 99.5) (width 1) (layer F.Cu) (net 4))
 (segment (start 142.2 99.5) (end 182.3 99.5) (width 2) (layer F.Cu) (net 4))
 (segment (start 182.3 99.5) (end 211.7 99.5) (width 2) (layer F.Cu) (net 4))
 (segment (start 210.9 93.4) (end 210.9 97) (width 1) (layer B.Cu) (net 4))
 (segment (start 216 97) (end 210.9 97) (width 2) (layer B.Cu) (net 4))
 (segment (start 210.9 97) (end 189.4 97) (width 2) (layer B.Cu) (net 4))
 (segment (start 131.1 93.4) (end 135.4 93.4) (width 1) (layer B.Cu) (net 4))
 (via (at 137 95) (size 0.8) (drill 0.4) (layers F.Cu B.Cu) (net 4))
 (segment (start 135.4 93.4) (end 137 95) (width 1) (layer B.Cu) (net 4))
 (segment (start 137 95) (end 138.6 93.4) (width 1) (layer F.Cu) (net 4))
 (segment (start 138.6 93.4) (end 142 93.4) (width 1) (layer F.Cu) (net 4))
 (segment (start 175.489998 93.4) (end 177.089998 95) (width 1) (layer B.Cu) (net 4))
 (segment (start 171 93.4) (end 175.489998 93.4) (width 1) (layer B.Cu) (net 4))
 (via (at 178 95) (size 0.8) (drill 0.4) (layers F.Cu B.Cu) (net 4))
 (segment (start 177.089998 95) (end 178 95) (width 1) (layer B.Cu) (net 4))
 (segment (start 178 95) (end 179.5 93.5) (width 1) (layer F.Cu) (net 4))
 (segment (start 179.6 93.4) (end 179.5 93.5) (width 1) (layer F.Cu) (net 4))
 (segment (start 181.9 93.4) (end 179.6 93.4) (width 1) (layer F.Cu) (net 4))
 (segment (start 117.8 93.4) (end 128.7 93.4) (width 1) (layer F.Cu) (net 17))
 (segment (start 128.5 96) (end 128 96) (width 1) (layer F.Cu) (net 18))
 (segment (start 131.1 93.4) (end 128.5 96) (width 1) (layer F.Cu) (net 18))
 (segment (start 144.4 93.4) (end 155.3 93.4) (width 1) (layer F.Cu) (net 16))
 (segment (start 157.7 93.4) (end 168.6 93.4) (width 1) (layer F.Cu) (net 14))
 (segment (start 168.4 96) (end 167.9 96) (width 1) (layer F.Cu) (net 15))
 (segment (start 171 93.4) (end 168.4 96) (width 1) (layer F.Cu) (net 15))
 (segment (start 184.3 93.4) (end 195.2 93.4) (width 1) (layer F.Cu) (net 13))
 (segment (start 197.6 93.4) (end 208.5 93.4) (width 1) (layer F.Cu) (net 11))
 (segment (start 208.3 96) (end 210.9 93.4) (width 1) (layer F.Cu) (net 12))
 (segment (start 207.2 96) (end 208.3 96) (width 1) (layer F.Cu) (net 12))
 (segment (start 197.6 93.4) (end 208.5 93.4) (width 1) (layer B.Cu) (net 10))
 (segment (start 184.3 93.4) (end 195.2 93.4) (width 1) (layer B.Cu) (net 8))
 (segment (start 184.5 96) (end 185.2 96) (width 1) (layer B.Cu) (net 9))
 (segment (start 181.9 93.4) (end 184.5 96) (width 1) (layer B.Cu) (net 9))
 (segment (start 157.7 93.4) (end 168.6 93.4) (width 1) (layer B.Cu) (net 7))
 (segment (start 144.4 93.4) (end 155.3 93.4) (width 1) (layer B.Cu) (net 5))
 (segment (start 144.6 96) (end 145.4 96) (width 1) (layer B.Cu) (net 6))
 (segment (start 142 93.4) (end 144.6 96) (width 1) (layer B.Cu) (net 6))
 (segment (start 117.8 93.4) (end 128.7 93.4) (width 1) (layer B.Cu) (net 3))
 (segment (start 104.5 93.4) (end 115.4 93.4) (width 1) (layer B.Cu) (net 1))
 (segment (start 102.1 93.4) (end 102.2 93.4) (width 1) (layer B.Cu) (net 2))
 (segment (start 104.8 96) (end 105.9 96) (width 1) (layer B.Cu) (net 2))
 (segment (start 102.2 93.4) (end 104.8 96) (width 1) (layer B.Cu) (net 2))
 (segment (start 97 99.54) (end 98.14 99.54) (width 2) (layer B.Cu) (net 20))
 (segment (start 98.14 99.54) (end 100.5 101.9) (width 2) (layer B.Cu) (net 20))
 (segment (start 100.5 101.9) (end 187.9 101.9) (width 2) (layer B.Cu) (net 20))
 (segment (start 190.26 99.54) (end 216 99.54) (width 2) (layer B.Cu) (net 20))
 (segment (start 187.9 101.9) (end 190.26 99.54) (width 2) (layer B.Cu) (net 20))
 (segment (start 97 99.54) (end 95.14 99.54) (width 2) (layer B.Cu) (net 20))
 (segment (start 95.14 99.54) (end 94.2 98.6) (width 2) (layer B.Cu) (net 20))
 (segment (start 94.2 98.6) (end 94.2 95.4) (width 2) (layer B.Cu) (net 20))
 (segment (start 94.2 95.4) (end 95.2 94.4) (width 2) (layer B.Cu) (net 20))
 (segment (start 95.2 94.4) (end 99.5 94.4) (width 2) (layer B.Cu) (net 20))
 (segment (start 101.1 96) (end 99.5 94.4) (width 1) (layer B.Cu) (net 20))
 (segment (start 101.9 96) (end 101.1 96) (width 1) (layer B.Cu) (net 20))
 (segment (start 102.05 96) (end 103.85 97.8) (width 1) (layer B.Cu) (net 20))
 (segment (start 101.9 96) (end 102.05 96) (width 1) (layer B.Cu) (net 20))
 (segment (start 179.4 97.8) (end 181.2 96) (width 1) (layer B.Cu) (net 20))
 (segment (start 141.4 97.7) (end 141.5 97.8) (width 1) (layer B.Cu) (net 20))
 (segment (start 141.4 96) (end 141.4 97.7) (width 1) (layer B.Cu) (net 20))
 (segment (start 215.128717 99.54) (end 215.1 99.568717) (width 2) (layer F.Cu) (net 20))
 (segment (start 216 99.54) (end 215.128717 99.54) (width 2) (layer F.Cu) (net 20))
 (segment (start 215.1 99.568717) (end 214.831283 99.568717) (width 2) (layer F.Cu) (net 20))
 (segment (start 214.831283 99.568717) (end 212.6 101.8) (width 2) (layer F.Cu) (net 20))
 (segment (start 97.871283 99.54) (end 97 99.54) (width 2) (layer F.Cu) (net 20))
 (segment (start 212.6 101.8) (end 100.131283 101.8) (width 2) (layer F.Cu) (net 20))
 (segment (start 100.131283 101.8) (end 97.871283 99.54) (width 2) (layer F.Cu) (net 20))
 (segment (start 211.2 96) (end 212.1 96) (width 1) (layer F.Cu) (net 20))
 (segment (start 212.1 96) (end 213.4 94.7) (width 1) (layer F.Cu) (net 20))
 (segment (start 213.4 94.7) (end 217.8 94.7) (width 1) (layer F.Cu) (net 20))
 (segment (start 217.8 94.7) (end 218.6 95.5) (width 1) (layer F.Cu) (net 20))
 (segment (start 218.6 95.5) (end 218.6 98.4) (width 1) (layer F.Cu) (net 20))
 (segment (start 217.46 99.54) (end 216 99.54) (width 1) (layer F.Cu) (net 20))
 (segment (start 218.6 98.4) (end 217.46 99.54) (width 1) (layer F.Cu) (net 20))
 (via (at 135 96) (size 0.8) (drill 0.4) (layers F.Cu B.Cu) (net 20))
 (segment (start 132 96) (end 135 96) (width 1) (layer F.Cu) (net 20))
 (segment (start 103.85 97.8) (end 134.9 97.8) (width 1) (layer B.Cu) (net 20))
 (segment (start 135 97.7) (end 134.9 97.8) (width 1) (layer B.Cu) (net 20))
 (segment (start 135 96) (end 135 97.7) (width 1) (layer B.Cu) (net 20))
 (segment (start 134.9 97.8) (end 141.5 97.8) (width 1) (layer B.Cu) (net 20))
 (segment (start 171.9 96) (end 176 96) (width 1) (layer F.Cu) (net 20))
 (via (at 176 96) (size 0.8) (drill 0.4) (layers F.Cu B.Cu) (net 20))
 (segment (start 176 96) (end 176 97.8) (width 1) (layer B.Cu) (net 20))
 (segment (start 141.5 97.8) (end 176 97.8) (width 1) (layer B.Cu) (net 20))
 (segment (start 176 97.8) (end 179.4 97.8) (width 1) (layer B.Cu) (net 20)))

